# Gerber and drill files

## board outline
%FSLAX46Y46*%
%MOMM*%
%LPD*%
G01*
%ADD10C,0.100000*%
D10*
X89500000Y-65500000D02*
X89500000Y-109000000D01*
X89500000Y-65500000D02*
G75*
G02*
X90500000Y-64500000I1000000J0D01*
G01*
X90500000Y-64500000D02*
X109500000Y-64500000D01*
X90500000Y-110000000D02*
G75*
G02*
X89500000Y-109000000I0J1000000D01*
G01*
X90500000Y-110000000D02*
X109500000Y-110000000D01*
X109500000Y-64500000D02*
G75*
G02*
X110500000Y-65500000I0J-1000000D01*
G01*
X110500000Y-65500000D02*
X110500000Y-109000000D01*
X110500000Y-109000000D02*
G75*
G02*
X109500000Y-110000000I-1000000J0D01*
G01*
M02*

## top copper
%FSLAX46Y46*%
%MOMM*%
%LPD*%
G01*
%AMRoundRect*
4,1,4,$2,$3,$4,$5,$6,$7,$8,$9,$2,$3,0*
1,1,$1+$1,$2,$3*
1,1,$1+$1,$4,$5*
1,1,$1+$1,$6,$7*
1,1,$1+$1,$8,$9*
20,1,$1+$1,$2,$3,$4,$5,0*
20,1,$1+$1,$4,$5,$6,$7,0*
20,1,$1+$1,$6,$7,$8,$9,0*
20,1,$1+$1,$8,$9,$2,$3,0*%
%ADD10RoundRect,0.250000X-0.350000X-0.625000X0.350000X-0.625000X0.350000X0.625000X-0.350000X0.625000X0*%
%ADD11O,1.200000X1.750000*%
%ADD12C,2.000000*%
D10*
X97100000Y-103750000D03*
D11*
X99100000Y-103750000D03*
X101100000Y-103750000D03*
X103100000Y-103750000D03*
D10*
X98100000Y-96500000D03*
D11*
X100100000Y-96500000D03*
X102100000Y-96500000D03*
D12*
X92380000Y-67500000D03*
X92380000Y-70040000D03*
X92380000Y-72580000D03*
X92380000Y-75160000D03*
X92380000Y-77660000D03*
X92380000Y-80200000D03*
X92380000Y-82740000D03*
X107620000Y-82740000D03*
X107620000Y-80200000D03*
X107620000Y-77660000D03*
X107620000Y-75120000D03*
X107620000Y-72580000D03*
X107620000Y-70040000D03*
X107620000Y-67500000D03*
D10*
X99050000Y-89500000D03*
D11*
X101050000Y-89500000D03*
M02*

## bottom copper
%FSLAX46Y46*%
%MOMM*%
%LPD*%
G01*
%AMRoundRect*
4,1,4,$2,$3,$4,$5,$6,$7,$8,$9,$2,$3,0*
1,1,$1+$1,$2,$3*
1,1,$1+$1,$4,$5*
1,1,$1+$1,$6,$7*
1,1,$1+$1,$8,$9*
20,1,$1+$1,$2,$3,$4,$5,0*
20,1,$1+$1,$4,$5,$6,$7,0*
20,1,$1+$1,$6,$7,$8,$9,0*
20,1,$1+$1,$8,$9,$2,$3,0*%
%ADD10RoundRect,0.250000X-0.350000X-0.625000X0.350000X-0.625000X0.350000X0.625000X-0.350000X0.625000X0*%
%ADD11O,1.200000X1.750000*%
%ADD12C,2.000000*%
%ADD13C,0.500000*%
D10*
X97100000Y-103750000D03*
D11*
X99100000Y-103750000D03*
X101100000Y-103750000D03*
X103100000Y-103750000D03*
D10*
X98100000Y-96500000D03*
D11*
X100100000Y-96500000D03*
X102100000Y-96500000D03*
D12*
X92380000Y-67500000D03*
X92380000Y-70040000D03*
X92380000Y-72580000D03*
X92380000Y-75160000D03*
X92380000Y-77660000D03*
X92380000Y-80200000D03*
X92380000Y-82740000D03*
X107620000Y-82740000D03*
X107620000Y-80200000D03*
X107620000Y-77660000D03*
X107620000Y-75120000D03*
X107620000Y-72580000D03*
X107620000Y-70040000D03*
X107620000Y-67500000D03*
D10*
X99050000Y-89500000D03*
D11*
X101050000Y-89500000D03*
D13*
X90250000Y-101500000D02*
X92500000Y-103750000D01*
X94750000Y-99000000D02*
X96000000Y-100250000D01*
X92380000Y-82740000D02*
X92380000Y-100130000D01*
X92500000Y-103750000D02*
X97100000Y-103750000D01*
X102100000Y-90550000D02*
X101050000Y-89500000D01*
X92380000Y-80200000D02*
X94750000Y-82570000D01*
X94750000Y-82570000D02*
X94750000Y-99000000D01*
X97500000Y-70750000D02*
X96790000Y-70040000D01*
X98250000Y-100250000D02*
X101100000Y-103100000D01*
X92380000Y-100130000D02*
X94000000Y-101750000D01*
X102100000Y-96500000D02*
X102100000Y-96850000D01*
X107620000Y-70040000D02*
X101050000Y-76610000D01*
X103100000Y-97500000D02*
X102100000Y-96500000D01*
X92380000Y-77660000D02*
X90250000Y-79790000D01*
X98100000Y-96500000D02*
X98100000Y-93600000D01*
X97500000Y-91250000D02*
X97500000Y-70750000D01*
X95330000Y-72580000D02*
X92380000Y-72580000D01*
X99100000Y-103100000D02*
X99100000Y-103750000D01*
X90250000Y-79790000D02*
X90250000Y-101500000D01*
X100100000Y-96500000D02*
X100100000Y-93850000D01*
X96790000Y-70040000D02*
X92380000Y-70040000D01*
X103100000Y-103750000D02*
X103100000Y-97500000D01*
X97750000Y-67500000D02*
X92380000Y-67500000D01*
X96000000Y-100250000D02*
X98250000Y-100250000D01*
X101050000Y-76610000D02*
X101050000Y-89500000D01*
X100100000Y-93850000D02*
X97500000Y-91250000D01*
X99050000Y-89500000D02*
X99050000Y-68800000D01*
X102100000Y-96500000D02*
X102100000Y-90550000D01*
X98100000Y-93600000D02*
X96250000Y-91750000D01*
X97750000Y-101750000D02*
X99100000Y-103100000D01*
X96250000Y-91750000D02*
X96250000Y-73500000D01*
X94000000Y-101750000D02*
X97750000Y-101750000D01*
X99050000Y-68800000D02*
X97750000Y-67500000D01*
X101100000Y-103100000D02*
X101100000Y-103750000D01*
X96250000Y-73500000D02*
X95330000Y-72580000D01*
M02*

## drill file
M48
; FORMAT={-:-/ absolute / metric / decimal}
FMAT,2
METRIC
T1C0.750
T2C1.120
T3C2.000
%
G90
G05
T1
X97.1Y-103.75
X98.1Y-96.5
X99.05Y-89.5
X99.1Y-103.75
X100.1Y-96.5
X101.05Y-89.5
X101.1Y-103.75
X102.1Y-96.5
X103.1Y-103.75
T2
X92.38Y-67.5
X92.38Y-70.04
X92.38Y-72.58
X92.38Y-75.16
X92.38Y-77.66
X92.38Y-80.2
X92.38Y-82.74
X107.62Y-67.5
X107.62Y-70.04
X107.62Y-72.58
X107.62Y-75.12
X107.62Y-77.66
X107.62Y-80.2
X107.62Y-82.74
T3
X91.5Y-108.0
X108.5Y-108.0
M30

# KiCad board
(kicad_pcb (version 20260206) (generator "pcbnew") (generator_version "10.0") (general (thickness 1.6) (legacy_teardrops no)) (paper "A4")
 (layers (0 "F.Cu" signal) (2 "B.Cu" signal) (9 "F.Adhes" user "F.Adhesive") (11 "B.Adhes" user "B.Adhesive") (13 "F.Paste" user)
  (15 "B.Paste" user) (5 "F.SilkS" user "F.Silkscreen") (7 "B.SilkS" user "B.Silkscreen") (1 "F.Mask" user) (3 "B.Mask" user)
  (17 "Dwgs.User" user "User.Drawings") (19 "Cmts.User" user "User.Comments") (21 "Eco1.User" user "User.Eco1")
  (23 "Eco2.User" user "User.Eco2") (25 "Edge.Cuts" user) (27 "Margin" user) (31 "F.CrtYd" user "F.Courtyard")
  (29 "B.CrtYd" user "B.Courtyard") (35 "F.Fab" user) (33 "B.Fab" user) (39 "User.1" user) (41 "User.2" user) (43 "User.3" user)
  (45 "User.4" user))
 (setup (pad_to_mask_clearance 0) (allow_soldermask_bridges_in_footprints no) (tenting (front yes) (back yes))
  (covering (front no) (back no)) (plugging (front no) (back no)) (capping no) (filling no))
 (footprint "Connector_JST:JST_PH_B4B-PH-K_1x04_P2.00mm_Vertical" (layer "F.Cu") (at 97.1 103.75)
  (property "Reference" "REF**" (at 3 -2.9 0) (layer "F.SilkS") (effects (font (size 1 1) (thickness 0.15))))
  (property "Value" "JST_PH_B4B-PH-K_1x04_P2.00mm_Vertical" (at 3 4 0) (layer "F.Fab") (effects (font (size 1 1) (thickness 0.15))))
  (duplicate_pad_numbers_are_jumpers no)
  (pad "1" thru_hole roundrect (at 0 0) (size 1.2 1.75) (drill 0.75) (layers "*.Cu" "*.Mask") (remove_unused_layers no)
   (roundrect_rratio 0.208333))
  (pad "2" thru_hole oval (at 2 0) (size 1.2 1.75) (drill 0.75) (layers "*.Cu" "*.Mask") (remove_unused_layers no))
  (pad "3" thru_hole oval (at 4 0) (size 1.2 1.75) (drill 0.75) (layers "*.Cu" "*.Mask") (remove_unused_layers no))
  (pad "4" thru_hole oval (at 6 0) (size 1.2 1.75) (drill 0.75) (layers "*.Cu" "*.Mask") (remove_unused_layers no)))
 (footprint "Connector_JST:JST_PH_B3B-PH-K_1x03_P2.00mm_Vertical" (layer "F.Cu") (at 98.1 96.5)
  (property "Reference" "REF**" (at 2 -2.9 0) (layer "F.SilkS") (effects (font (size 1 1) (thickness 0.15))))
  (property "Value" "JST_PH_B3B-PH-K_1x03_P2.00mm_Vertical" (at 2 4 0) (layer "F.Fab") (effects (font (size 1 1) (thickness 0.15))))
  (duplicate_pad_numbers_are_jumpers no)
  (pad "1" thru_hole roundrect (at 0 0) (size 1.2 1.75) (drill 0.75) (layers "*.Cu" "*.Mask") (remove_unused_layers no)
   (roundrect_rratio 0.208333))
  (pad "2" thru_hole oval (at 2 0) (size 1.2 1.75) (drill 0.75) (layers "*.Cu" "*.Mask") (remove_unused_layers no))
  (pad "3" thru_hole oval (at 4 0) (size 1.2 1.75) (drill 0.75) (layers "*.Cu" "*.Mask") (remove_unused_layers no)))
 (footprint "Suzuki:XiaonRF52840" (layer "F.Cu") (at 100 75.12 -90)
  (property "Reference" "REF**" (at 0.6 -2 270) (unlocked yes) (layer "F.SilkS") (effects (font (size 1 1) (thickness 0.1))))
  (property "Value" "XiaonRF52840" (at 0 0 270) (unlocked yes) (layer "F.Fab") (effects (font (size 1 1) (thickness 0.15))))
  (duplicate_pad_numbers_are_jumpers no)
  (pad "1" thru_hole circle (at -7.62 7.62 270) (size 2 2) (drill 1.12) (layers "*.Cu" "*.Mask") (remove_unused_layers no))
  (pad "2" thru_hole circle (at -5.08 7.62 270) (size 2 2) (drill 1.12) (layers "*.Cu" "*.Mask") (remove_unused_layers no))
  (pad "3" thru_hole circle (at -2.54 7.62 270) (size 2 2) (drill 1.12) (layers "*.Cu" "*.Mask") (remove_unused_layers no))
  (pad "4" thru_hole circle (at 0.04 7.62 270) (size 2 2) (drill 1.12) (layers "*.Cu" "*.Mask") (remove_unused_layers no))
  (pad "5" thru_hole circle (at 2.54 7.62 270) (size 2 2) (drill 1.12) (layers "*.Cu" "*.Mask") (remove_unused_layers no))
  (pad "6" thru_hole circle (at 5.08 7.62 270) (size 2 2) (drill 1.12) (layers "*.Cu" "*.Mask") (remove_unused_layers no))
  (pad "7" thru_hole circle (at 7.62 7.62 270) (size 2 2) (drill 1.12) (layers "*.Cu" "*.Mask") (remove_unused_layers no))
  (pad "8" thru_hole circle (at 7.62 -7.62 270) (size 2 2) (drill 1.12) (layers "*.Cu" "*.Mask") (remove_unused_layers no))
  (pad "9" thru_hole circle (at 5.08 -7.62 270) (size 2 2) (drill 1.12) (layers "*.Cu" "*.Mask") (remove_unused_layers no))
  (pad "10" thru_hole circle (at 2.54 -7.62 270) (size 2 2) (drill 1.12) (layers "*.Cu" "*.Mask") (remove_unused_layers no))
  (pad "11" thru_hole circle (at 0 -7.62 270) (size 2 2) (drill 1.12) (layers "*.Cu" "*.Mask") (remove_unused_layers no))
  (pad "12" thru_hole circle (at -2.54 -7.62 270) (size 2 2) (drill 1.12) (layers "*.Cu" "*.Mask") (remove_unused_layers no))
  (pad "13" thru_hole circle (at -5.08 -7.62 270) (size 2 2) (drill 1.12) (layers "*.Cu" "*.Mask") (remove_unused_layers no))
  (pad "14" thru_hole circle (at -7.62 -7.62 270) (size 2 2) (drill 1.12) (layers "*.Cu" "*.Mask") (remove_unused_layers no)))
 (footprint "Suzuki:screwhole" (layer "F.Cu") (at 108.75 108)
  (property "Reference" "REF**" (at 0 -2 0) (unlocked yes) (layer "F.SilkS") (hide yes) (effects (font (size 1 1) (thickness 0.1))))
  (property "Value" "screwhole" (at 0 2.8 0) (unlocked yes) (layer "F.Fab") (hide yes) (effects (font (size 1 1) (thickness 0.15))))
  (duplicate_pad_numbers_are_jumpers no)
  (pad "" np_thru_hole circle (at -0.25 0) (size 2 2) (drill 2) (layers "*.Cu" "*.Mask")))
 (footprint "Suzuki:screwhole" (layer "F.Cu") (at 91.5 108)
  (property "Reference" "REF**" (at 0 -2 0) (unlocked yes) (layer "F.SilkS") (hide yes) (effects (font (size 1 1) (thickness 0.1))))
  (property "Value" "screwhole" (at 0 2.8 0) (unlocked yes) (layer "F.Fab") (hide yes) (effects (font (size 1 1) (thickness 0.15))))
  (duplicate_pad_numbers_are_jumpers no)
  (pad "" np_thru_hole circle (at 0 0) (size 2 2) (drill 2) (layers "*.Cu" "*.Mask")))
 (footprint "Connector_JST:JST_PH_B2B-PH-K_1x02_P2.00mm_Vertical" (layer "F.Cu") (at 99.05 89.5)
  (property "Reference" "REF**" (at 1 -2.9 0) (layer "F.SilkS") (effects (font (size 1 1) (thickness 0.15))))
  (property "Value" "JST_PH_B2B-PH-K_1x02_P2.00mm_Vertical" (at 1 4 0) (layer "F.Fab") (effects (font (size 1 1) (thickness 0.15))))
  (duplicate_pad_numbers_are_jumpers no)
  (pad "1" thru_hole roundrect (at 0 0) (size 1.2 1.75) (drill 0.75) (layers "*.Cu" "*.Mask") (remove_unused_layers no)
   (roundrect_rratio 0.208333))
  (pad "2" thru_hole oval (at 2 0) (size 1.2 1.75) (drill 0.75) (layers "*.Cu" "*.Mask") (remove_unused_layers no)))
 (gr_line (start 89.5 65.5) (end 89.5 109) (stroke (width 0.1) (type solid)) (layer "Edge.Cuts"))
 (gr_arc (start 89.5 65.5) (mid 89.792893 64.792893) (end 90.5 64.5) (stroke (width 0.1) (type default)) (layer "Edge.Cuts"))
 (gr_line (start 90.5 64.5) (end 109.5 64.5) (stroke (width 0.1) (type solid)) (layer "Edge.Cuts"))
 (gr_arc (start 90.5 110) (mid 89.792893 109.707107) (end 89.5 109) (stroke (width 0.1) (type default)) (layer "Edge.Cuts"))
 (gr_line (start 90.5 110) (end 109.5 110) (stroke (width 0.1) (type solid)) (layer "Edge.Cuts"))
 (gr_arc (start 109.5 64.5) (mid 110.207107 64.792893) (end 110.5 65.5) (stroke (width 0.1) (type default)) (layer "Edge.Cuts"))
 (gr_line (start 110.5 65.5) (end 110.5 109) (stroke (width 0.1) (type solid)) (layer "Edge.Cuts"))
 (gr_arc (start 110.5 109) (mid 110.207107 109.707107) (end 109.5 110) (stroke (width 0.1) (type default)) (layer "Edge.Cuts"))
 (segment (start 90.25 101.5) (end 92.5 103.75) (width 0.5) (layer "B.Cu") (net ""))
 (segment (start 94.75 99) (end 96 100.25) (width 0.5) (layer "B.Cu") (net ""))
 (segment (start 92.38 82.74) (end 92.38 100.13) (width 0.5) (layer "B.Cu") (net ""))
 (segment (start 92.5 103.75) (end 97.1 103.75) (width 0.5) (layer "B.Cu") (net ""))
 (segment (start 102.1 90.55) (end 101.05 89.5) (width 0.5) (layer "B.Cu") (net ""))
 (segment (start 92.38 80.2) (end 94.75 82.57) (width 0.5) (layer "B.Cu") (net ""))
 (segment (start 94.75 82.57) (end 94.75 99) (width 0.5) (layer "B.Cu") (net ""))
 (segment (start 97.5 70.75) (end 96.79 70.04) (width 0.5) (layer "B.Cu") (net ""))
 (segment (start 98.25 100.25) (end 101.1 103.1) (width 0.5) (layer "B.Cu") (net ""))
 (segment (start 92.38 100.13) (end 94 101.75) (width 0.5) (layer "B.Cu") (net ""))
 (segment (start 102.1 96.5) (end 102.1 96.85) (width 0.5) (layer "B.Cu") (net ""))
 (segment (start 107.62 70.04) (end 101.05 76.61) (width 0.5) (layer "B.Cu") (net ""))
 (segment (start 103.1 97.5) (end 102.1 96.5) (width 0.5) (layer "B.Cu") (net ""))
 (segment (start 92.38 77.66) (end 90.25 79.79) (width 0.5) (layer "B.Cu") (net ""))
 (segment (start 98.1 96.5) (end 98.1 93.6) (width 0.5) (layer "B.Cu") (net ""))
 (segment (start 97.5 91.25) (end 97.5 70.75) (width 0.5) (layer "B.Cu") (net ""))
 (segment (start 95.33 72.58) (end 92.38 72.58) (width 0.5) (layer "B.Cu") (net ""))
 (segment (start 99.1 103.1) (end 99.1 103.75) (width 0.5) (layer "B.Cu") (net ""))
 (segment (start 90.25 79.79) (end 90.25 101.5) (width 0.5) (layer "B.Cu") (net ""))
 (segment (start 100.1 96.5) (end 100.1 93.85) (width 0.5) (layer "B.Cu") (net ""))
 (segment (start 96.79 70.04) (end 92.38 70.04) (width 0.5) (layer "B.Cu") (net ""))
 (segment (start 103.1 103.75) (end 103.1 97.5) (width 0.5) (layer "B.Cu") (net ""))
 (segment (start 97.75 67.5) (end 92.38 67.5) (width 0.5) (layer "B.Cu") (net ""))
 (segment (start 96 100.25) (end 98.25 100.25) (width 0.5) (layer "B.Cu") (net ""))
 (segment (start 101.05 76.61) (end 101.05 89.5) (width 0.5) (layer "B.Cu") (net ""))
 (segment (start 100.1 93.85) (end 97.5 91.25) (width 0.5) (layer "B.Cu") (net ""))
 (segment (start 99.05 89.5) (end 99.05 68.8) (width 0.5) (layer "B.Cu") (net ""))
 (segment (start 102.1 96.5) (end 102.1 90.55) (width 0.5) (layer "B.Cu") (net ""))
 (segment (start 98.1 93.6) (end 96.25 91.75) (width 0.5) (layer "B.Cu") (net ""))
 (segment (start 97.75 101.75) (end 99.1 103.1) (width 0.5) (layer "B.Cu") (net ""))
 (segment (start 96.25 91.75) (end 96.25 73.5) (width 0.5) (layer "B.Cu") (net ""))
 (segment (start 94 101.75) (end 97.75 101.75) (width 0.5) (layer "B.Cu") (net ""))
 (segment (start 99.05 68.8) (end 97.75 67.5) (width 0.5) (layer "B.Cu") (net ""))
 (segment (start 101.1 103.1) (end 101.1 103.75) (width 0.5) (layer "B.Cu") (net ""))
 (segment (start 96.25 73.5) (end 95.33 72.58) (width 0.5) (layer "B.Cu") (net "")))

